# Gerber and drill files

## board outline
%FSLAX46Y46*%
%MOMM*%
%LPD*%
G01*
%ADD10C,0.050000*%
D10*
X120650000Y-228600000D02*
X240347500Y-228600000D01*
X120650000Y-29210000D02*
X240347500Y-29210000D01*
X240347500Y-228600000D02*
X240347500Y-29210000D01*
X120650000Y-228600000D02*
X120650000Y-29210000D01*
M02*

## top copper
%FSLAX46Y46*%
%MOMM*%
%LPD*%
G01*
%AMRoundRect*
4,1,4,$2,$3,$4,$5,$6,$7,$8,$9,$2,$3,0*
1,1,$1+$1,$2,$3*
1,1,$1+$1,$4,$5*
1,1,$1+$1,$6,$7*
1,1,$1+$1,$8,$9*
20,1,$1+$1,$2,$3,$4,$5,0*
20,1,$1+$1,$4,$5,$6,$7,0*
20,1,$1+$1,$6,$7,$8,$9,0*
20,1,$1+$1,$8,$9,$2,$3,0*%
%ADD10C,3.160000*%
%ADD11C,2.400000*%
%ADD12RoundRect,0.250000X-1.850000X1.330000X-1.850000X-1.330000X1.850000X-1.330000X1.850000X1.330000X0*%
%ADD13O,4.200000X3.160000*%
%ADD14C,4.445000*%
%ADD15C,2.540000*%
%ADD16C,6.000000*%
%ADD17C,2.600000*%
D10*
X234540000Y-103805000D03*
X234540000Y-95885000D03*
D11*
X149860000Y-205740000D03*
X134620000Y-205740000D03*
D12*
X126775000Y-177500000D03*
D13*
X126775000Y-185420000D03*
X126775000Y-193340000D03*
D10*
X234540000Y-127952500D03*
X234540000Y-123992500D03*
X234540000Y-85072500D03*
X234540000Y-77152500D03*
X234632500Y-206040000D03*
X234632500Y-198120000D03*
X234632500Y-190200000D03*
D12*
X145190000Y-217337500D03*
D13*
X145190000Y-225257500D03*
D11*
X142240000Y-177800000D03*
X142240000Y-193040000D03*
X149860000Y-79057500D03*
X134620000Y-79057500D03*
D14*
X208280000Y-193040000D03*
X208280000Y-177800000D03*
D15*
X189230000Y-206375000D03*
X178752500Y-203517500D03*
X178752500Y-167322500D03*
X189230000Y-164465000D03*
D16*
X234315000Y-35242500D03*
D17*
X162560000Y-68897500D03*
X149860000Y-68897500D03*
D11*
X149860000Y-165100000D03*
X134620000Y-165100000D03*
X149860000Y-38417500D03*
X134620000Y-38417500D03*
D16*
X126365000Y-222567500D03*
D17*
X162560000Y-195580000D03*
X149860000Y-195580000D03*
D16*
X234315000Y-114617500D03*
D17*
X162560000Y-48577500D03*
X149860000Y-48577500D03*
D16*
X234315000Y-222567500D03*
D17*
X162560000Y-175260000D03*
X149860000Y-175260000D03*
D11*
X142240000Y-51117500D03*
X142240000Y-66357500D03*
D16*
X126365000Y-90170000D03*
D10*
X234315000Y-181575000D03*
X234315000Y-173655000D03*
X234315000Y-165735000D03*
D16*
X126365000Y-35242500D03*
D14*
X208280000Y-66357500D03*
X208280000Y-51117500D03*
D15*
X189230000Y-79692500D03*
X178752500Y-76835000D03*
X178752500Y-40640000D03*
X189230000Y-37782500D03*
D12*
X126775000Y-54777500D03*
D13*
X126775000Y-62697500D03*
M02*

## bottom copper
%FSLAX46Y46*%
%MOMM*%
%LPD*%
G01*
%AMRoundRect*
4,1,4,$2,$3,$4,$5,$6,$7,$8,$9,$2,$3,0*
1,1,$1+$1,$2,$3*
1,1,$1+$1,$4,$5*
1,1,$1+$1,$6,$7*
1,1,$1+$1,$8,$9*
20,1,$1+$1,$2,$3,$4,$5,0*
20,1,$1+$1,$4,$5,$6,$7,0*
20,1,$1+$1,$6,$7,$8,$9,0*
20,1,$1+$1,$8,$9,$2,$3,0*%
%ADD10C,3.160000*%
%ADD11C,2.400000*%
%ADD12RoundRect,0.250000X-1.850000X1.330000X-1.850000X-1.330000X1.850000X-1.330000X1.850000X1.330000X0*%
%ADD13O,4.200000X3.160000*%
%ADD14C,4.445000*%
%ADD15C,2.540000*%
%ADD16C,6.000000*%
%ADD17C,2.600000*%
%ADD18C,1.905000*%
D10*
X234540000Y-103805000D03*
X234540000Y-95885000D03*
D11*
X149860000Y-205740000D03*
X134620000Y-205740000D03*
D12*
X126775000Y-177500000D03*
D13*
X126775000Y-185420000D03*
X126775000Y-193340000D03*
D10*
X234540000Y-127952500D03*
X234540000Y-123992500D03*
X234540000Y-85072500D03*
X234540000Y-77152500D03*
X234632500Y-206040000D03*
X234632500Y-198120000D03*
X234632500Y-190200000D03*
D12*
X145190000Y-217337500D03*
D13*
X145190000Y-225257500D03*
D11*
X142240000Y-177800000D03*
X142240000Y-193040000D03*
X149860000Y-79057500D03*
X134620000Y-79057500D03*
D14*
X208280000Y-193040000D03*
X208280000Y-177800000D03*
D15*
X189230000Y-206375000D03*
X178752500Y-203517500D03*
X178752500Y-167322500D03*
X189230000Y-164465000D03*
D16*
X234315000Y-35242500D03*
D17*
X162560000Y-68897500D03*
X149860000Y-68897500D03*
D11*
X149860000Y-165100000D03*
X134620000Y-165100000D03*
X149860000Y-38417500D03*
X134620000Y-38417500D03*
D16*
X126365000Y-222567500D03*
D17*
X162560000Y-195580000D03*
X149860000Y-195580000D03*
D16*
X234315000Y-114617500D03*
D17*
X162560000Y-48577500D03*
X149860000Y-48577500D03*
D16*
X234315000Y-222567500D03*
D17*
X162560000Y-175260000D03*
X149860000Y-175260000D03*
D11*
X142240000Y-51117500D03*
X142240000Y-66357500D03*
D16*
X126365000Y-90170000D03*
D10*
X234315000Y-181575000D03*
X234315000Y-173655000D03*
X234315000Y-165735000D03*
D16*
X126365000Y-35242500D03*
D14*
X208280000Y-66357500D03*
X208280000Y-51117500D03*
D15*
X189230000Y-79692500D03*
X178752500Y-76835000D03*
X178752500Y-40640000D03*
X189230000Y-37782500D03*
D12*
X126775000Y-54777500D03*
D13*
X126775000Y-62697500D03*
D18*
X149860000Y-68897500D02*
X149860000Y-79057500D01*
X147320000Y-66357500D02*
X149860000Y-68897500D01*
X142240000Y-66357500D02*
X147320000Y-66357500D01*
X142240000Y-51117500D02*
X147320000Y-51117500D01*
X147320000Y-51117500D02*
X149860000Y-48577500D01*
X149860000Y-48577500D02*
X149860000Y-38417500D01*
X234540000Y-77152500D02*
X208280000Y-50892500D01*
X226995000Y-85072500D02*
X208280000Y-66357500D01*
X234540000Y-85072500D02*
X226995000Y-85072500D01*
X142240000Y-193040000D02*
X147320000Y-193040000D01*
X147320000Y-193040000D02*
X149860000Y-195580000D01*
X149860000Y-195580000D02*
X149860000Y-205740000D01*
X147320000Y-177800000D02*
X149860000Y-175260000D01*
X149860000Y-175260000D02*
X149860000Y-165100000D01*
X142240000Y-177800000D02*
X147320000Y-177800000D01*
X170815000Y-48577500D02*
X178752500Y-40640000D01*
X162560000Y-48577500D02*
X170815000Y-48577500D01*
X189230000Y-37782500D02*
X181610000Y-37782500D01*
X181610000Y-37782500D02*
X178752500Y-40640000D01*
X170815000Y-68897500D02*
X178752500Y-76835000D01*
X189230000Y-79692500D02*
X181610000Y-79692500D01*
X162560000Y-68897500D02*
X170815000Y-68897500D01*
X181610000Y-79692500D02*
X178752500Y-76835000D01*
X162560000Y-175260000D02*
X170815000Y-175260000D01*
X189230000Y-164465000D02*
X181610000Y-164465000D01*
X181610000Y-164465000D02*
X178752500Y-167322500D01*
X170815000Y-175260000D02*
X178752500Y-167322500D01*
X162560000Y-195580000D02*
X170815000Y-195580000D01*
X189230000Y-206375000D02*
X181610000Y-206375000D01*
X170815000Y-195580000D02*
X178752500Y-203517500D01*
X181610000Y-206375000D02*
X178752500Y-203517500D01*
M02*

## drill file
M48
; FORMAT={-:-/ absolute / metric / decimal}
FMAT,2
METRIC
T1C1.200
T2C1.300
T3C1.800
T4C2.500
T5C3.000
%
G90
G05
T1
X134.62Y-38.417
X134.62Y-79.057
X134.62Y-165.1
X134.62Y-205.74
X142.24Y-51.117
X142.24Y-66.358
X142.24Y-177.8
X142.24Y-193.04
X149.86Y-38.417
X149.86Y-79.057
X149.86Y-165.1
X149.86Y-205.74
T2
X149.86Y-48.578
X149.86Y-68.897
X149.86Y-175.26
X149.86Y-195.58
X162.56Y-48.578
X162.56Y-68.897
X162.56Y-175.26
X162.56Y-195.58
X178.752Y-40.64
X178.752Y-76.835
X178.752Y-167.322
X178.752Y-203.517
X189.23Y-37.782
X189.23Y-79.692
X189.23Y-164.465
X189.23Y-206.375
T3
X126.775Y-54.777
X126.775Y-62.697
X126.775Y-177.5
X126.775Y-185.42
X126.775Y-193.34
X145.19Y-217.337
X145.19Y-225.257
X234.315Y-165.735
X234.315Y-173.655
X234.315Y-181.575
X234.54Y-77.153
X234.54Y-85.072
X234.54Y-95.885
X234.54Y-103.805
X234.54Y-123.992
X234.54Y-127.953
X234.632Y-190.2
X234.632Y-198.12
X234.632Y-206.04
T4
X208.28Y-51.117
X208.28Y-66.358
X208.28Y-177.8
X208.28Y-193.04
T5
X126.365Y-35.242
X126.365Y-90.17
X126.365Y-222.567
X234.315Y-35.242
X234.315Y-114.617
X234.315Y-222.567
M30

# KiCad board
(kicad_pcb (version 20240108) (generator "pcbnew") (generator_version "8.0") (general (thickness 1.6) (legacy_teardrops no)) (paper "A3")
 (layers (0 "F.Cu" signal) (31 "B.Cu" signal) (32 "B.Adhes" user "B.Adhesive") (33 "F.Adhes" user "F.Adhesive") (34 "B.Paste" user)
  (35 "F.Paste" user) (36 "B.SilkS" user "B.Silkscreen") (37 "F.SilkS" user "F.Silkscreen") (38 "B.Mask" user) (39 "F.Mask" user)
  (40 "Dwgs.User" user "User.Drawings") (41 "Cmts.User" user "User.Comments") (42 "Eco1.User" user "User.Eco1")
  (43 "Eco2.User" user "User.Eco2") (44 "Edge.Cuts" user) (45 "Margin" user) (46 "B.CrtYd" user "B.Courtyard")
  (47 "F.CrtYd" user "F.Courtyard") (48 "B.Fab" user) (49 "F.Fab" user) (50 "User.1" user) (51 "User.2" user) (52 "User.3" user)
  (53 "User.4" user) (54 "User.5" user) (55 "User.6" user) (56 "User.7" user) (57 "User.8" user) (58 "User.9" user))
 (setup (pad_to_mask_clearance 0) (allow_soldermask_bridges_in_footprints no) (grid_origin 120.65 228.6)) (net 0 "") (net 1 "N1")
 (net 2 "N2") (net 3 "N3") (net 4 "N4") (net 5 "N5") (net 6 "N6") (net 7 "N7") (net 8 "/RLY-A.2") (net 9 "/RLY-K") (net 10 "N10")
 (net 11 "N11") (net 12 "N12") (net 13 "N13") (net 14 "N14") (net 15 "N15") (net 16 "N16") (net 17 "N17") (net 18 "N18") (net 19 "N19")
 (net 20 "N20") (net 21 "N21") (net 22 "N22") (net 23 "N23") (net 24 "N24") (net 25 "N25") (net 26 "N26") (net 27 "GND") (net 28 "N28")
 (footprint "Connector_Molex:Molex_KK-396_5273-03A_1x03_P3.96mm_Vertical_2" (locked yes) (layer "F.Cu") (at 234.54 103.805 90)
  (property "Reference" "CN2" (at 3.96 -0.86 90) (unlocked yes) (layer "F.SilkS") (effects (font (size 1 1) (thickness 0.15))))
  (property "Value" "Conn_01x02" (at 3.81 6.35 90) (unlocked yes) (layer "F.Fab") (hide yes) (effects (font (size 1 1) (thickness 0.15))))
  (pad "1" thru_hole circle (at 0 0 90) (size 3.16 3.16) (drill 1.8) (layers "*.Cu" "*.Mask") (remove_unused_layers no) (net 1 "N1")
   (thermal_bridge_angle 90))
  (pad "2" thru_hole circle (at 7.92 0 90) (size 3.16 3.16) (drill 1.8) (layers "*.Cu" "*.Mask") (remove_unused_layers no) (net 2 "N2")
   (thermal_bridge_angle 90)))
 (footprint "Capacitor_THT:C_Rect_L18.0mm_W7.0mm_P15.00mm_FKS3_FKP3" (layer "F.Cu") (at 142.24 205.74 180)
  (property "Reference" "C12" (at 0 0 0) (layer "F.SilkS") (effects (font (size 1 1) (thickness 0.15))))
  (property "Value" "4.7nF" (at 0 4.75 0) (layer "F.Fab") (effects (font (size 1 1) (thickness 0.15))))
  (pad "1" thru_hole circle (at -7.62 0 180) (size 2.4 2.4) (drill 1.2) (layers "*.Cu" "*.Mask") (remove_unused_layers no) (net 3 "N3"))
  (pad "2" thru_hole circle (at 7.62 0 180) (size 2.4 2.4) (drill 1.2) (layers "*.Cu" "*.Mask") (remove_unused_layers no) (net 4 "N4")))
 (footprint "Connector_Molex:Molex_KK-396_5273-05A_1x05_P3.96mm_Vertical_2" (layer "F.Cu") (at 126.775 177.5 -90)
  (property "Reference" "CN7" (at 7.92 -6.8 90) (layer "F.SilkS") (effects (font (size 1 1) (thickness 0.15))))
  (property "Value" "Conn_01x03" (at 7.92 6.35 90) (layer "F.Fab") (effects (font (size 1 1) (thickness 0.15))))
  (pad "1" thru_hole roundrect (at 0 0 270) (size 3.16 4.2) (drill 1.8) (layers "*.Cu" "*.Mask") (remove_unused_layers no)
   (roundrect_rratio 0.079114) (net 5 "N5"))
  (pad "2" thru_hole oval (at 7.92 0 270) (size 3.16 4.2) (drill 1.8) (layers "*.Cu" "*.Mask") (remove_unused_layers no) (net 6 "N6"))
  (pad "3" thru_hole oval (at 15.84 0 270) (size 3.16 4.2) (drill 1.8) (layers "*.Cu" "*.Mask") (remove_unused_layers no) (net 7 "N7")))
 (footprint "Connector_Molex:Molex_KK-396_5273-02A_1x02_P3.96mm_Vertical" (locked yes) (layer "F.Cu") (at 234.54 127.9525 90)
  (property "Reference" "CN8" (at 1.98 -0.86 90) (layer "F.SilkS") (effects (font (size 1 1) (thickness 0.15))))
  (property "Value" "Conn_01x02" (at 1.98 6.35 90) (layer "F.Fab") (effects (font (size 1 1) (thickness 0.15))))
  (pad "1" thru_hole circle (at 0 0 90) (size 3.16 3.16) (drill 1.8) (layers "*.Cu" "*.Mask") (remove_unused_layers no) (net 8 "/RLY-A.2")
   (thermal_bridge_angle 90))
  (pad "2" thru_hole circle (at 3.96 0 90) (size 3.16 3.16) (drill 1.8) (layers "*.Cu" "*.Mask") (remove_unused_layers no) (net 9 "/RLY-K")
   (thermal_bridge_angle 90)))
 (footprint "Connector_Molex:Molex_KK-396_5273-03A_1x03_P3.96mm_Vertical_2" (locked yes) (layer "F.Cu") (at 234.54 85.0725 90)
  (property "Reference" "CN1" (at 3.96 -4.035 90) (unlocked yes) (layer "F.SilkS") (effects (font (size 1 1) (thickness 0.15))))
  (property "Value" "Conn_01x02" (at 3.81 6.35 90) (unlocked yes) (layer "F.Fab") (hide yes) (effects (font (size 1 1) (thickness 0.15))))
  (pad "1" thru_hole circle (at 0 0 90) (size 3.16 4.2) (drill 1.8) (layers "*.Cu" "*.Mask") (remove_unused_layers no) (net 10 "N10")
   (thermal_bridge_angle 90))
  (pad "2" thru_hole circle (at 7.92 0 90) (size 3.16 4.2) (drill 1.8) (layers "*.Cu" "*.Mask") (remove_unused_layers no) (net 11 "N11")
   (thermal_bridge_angle 90)))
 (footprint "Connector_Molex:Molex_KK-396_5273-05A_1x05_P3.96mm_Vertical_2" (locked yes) (layer "F.Cu") (at 234.6325 206.04 90)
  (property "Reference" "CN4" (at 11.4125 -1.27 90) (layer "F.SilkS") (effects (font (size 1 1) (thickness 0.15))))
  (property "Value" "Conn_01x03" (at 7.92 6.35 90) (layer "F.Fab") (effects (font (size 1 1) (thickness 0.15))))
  (pad "1" thru_hole circle (at 0 0 90) (size 3.16 4.2) (drill 1.8) (layers "*.Cu" "*.Mask") (remove_unused_layers no) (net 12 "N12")
   (thermal_bridge_angle 90))
  (pad "2" thru_hole circle (at 7.92 0 90) (size 3.16 4.2) (drill 1.8) (layers "*.Cu" "*.Mask") (remove_unused_layers no) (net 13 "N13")
   (thermal_bridge_angle 90))
  (pad "3" thru_hole circle (at 15.84 0 90) (size 3.16 4.2) (drill 1.8) (layers "*.Cu" "*.Mask") (remove_unused_layers no) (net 4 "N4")
   (thermal_bridge_angle 90)))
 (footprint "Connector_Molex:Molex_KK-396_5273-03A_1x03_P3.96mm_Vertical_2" (layer "F.Cu") (at 145.19 217.3375 -90)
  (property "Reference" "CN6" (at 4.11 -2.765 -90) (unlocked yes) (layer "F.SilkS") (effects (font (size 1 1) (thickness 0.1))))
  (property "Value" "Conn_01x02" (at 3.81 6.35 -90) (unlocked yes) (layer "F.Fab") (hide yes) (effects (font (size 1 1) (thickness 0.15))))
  (pad "1" thru_hole roundrect (at 0 0 270) (size 3.16 4.2) (drill 1.8) (layers "*.Cu" "*.Mask") (remove_unused_layers no)
   (roundrect_rratio 0.079114) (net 13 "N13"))
  (pad "2" thru_hole oval (at 7.92 0 270) (size 3.16 4.2) (drill 1.8) (layers "*.Cu" "*.Mask") (remove_unused_layers no) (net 12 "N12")))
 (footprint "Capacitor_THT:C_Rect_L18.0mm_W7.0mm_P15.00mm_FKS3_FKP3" (layer "F.Cu") (at 142.24 185.42 -90)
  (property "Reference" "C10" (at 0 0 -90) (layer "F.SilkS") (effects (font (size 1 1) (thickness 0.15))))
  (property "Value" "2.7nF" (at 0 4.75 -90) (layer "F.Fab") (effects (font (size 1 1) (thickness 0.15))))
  (pad "1" thru_hole circle (at -7.62 0 270) (size 2.4 2.4) (drill 1.2) (layers "*.Cu" "*.Mask") (remove_unused_layers no) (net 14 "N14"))
  (pad "2" thru_hole circle (at 7.62 0 270) (size 2.4 2.4) (drill 1.2) (layers "*.Cu" "*.Mask") (remove_unused_layers no) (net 3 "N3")))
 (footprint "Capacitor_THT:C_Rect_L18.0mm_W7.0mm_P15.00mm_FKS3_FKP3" (layer "F.Cu") (at 142.24 79.0575 180)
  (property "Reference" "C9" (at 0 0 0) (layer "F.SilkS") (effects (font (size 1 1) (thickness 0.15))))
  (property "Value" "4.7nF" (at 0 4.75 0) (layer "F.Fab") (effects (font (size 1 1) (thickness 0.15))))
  (pad "1" thru_hole circle (at -7.62 0 180) (size 2.4 2.4) (drill 1.2) (layers "*.Cu" "*.Mask") (remove_unused_layers no) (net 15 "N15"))
  (pad "2" thru_hole circle (at 7.62 0 180) (size 2.4 2.4) (drill 1.2) (layers "*.Cu" "*.Mask") (remove_unused_layers no) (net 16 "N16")))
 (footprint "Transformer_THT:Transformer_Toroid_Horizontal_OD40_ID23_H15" (layer "F.Cu") (at 189.23 185.42 90)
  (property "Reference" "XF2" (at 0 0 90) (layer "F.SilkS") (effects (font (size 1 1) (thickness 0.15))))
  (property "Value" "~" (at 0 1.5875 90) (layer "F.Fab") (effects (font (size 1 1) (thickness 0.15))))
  (pad "1" thru_hole circle (at -7.62 19.05 90) (size 4.445 2.54) (drill 2.5) (layers "*.Cu" "*.Mask") (remove_unused_layers no)
   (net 1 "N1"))
  (pad "2" thru_hole circle (at 7.62 19.05 90) (size 4.445 2.54) (drill 2.5) (layers "*.Cu" "*.Mask") (remove_unused_layers no) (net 2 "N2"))
  (pad "3" thru_hole circle (at -20.955 0 90) (size 2.54 2.54) (drill 1.3) (layers "*.Cu" "*.Mask") (remove_unused_layers no) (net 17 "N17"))
  (pad "3" thru_hole circle (at -18.0975 -10.4775 90) (size 2.54 2.54) (drill 1.3) (layers "*.Cu" "*.Mask") (remove_unused_layers no)
   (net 17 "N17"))
  (pad "4" thru_hole circle (at 18.0975 -10.4775 90) (size 2.54 2.54) (drill 1.3) (layers "*.Cu" "*.Mask") (remove_unused_layers no)
   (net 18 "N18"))
  (pad "4" thru_hole circle (at 20.955 0 90) (size 2.54 2.54) (drill 1.3) (layers "*.Cu" "*.Mask") (remove_unused_layers no) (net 18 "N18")))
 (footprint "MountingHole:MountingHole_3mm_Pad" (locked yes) (layer "F.Cu") (at 234.315 35.2425 -90)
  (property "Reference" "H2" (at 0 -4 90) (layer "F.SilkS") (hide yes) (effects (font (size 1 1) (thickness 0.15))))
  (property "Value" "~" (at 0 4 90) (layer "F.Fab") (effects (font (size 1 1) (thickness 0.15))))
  (pad "1" thru_hole circle (at 0 0 270) (size 6 6) (drill 3) (layers "*.Cu" "*.Mask") (remove_unused_layers no) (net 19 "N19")))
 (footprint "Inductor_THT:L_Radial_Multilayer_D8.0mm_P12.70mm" (layer "F.Cu") (at 158.115 68.8975 180)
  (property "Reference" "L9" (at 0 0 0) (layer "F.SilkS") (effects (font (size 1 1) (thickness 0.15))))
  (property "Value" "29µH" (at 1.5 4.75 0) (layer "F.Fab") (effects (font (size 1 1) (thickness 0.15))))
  (pad "1" thru_hole circle (at -4.445 0 180) (size 2.6 2.6) (drill 1.3) (layers "*.Cu" "*.Mask") (remove_unused_layers no) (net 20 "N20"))
  (pad "2" thru_hole circle (at 8.255 0 180) (size 2.6 2.6) (drill 1.3) (layers "*.Cu" "*.Mask") (remove_unused_layers no) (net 15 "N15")))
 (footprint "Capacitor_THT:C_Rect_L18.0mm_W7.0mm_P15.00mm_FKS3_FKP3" (layer "F.Cu") (at 142.24 165.1 180)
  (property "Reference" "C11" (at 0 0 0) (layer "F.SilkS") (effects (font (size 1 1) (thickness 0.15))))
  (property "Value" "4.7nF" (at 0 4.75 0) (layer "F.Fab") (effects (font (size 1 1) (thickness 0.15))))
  (pad "1" thru_hole circle (at -7.62 0 180) (size 2.4 2.4) (drill 1.2) (layers "*.Cu" "*.Mask") (remove_unused_layers no) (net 14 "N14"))
  (pad "2" thru_hole circle (at 7.62 0 180) (size 2.4 2.4) (drill 1.2) (layers "*.Cu" "*.Mask") (remove_unused_layers no) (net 7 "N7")))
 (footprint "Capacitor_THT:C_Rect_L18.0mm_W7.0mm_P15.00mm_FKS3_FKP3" (layer "F.Cu") (at 142.24 38.4175 180)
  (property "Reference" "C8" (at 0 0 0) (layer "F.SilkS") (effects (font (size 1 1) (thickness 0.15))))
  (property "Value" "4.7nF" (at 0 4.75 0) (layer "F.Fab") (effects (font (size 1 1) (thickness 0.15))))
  (pad "1" thru_hole circle (at -7.62 0 180) (size 2.4 2.4) (drill 1.2) (layers "*.Cu" "*.Mask") (remove_unused_layers no) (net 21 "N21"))
  (pad "2" thru_hole circle (at 7.62 0 180) (size 2.4 2.4) (drill 1.2) (layers "*.Cu" "*.Mask") (remove_unused_layers no) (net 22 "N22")))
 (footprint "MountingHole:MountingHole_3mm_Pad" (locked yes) (layer "F.Cu") (at 126.365 222.5675)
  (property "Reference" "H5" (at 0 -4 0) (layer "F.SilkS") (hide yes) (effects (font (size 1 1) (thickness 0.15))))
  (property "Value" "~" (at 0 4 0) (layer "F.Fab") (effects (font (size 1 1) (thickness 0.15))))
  (pad "1" thru_hole circle (at 0 0) (size 6 6) (drill 3) (layers "*.Cu" "*.Mask") (remove_unused_layers no) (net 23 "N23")))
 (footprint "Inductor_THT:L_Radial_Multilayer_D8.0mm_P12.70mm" (layer "F.Cu") (at 158.115 195.58 180)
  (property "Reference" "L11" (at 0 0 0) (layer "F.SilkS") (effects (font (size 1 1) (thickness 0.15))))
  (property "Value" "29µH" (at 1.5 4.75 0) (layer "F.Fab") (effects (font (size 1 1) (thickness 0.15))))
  (pad "1" thru_hole circle (at -4.445 0 180) (size 2.6 2.6) (drill 1.3) (layers "*.Cu" "*.Mask") (remove_unused_layers no) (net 17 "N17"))
  (pad "2" thru_hole circle (at 8.255 0 180) (size 2.6 2.6) (drill 1.3) (layers "*.Cu" "*.Mask") (remove_unused_layers no) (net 3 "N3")))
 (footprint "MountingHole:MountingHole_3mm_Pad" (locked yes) (layer "F.Cu") (at 234.315 114.6175 -90)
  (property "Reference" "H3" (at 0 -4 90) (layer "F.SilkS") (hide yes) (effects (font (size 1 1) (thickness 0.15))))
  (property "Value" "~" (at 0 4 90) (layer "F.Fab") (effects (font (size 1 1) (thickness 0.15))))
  (pad "1" thru_hole circle (at 0 0 270) (size 6 6) (drill 3) (layers "*.Cu" "*.Mask") (remove_unused_layers no) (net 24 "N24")))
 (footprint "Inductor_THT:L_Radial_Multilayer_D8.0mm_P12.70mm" (layer "F.Cu") (at 158.115 48.5775 180)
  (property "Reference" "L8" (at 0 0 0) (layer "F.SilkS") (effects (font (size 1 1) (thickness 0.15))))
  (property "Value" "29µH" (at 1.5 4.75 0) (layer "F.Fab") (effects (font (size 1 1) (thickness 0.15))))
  (pad "1" thru_hole circle (at -4.445 0 180) (size 2.6 2.6) (drill 1.3) (layers "*.Cu" "*.Mask") (remove_unused_layers no) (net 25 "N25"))
  (pad "2" thru_hole circle (at 8.255 0 180) (size 2.6 2.6) (drill 1.3) (layers "*.Cu" "*.Mask") (remove_unused_layers no) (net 21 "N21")))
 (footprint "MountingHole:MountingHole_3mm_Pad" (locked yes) (layer "F.Cu") (at 234.315 222.5675)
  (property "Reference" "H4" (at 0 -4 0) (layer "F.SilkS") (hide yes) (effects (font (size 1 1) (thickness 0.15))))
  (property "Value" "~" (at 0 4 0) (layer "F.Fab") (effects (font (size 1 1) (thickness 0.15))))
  (pad "1" thru_hole circle (at 0 0) (size 6 6) (drill 3) (layers "*.Cu" "*.Mask") (remove_unused_layers no) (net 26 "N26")))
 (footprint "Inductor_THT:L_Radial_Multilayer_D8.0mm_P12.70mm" (layer "F.Cu") (at 158.115 175.26 180)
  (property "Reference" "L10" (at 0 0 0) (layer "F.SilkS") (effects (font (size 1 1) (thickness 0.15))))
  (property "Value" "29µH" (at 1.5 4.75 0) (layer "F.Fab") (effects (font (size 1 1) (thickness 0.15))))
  (pad "1" thru_hole circle (at -4.445 0 180) (size 2.6 2.6) (drill 1.3) (layers "*.Cu" "*.Mask") (remove_unused_layers no) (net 18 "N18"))
  (pad "2" thru_hole circle (at 8.255 0 180) (size 2.6 2.6) (drill 1.3) (layers "*.Cu" "*.Mask") (remove_unused_layers no) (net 14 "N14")))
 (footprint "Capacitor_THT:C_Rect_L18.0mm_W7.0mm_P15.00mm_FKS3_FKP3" (layer "F.Cu") (at 142.24 58.7375 -90)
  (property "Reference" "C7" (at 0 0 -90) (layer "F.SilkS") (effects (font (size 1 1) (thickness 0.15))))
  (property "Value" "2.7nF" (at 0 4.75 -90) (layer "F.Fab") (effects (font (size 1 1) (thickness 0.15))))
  (pad "1" thru_hole circle (at -7.62 0 270) (size 2.4 2.4) (drill 1.2) (layers "*.Cu" "*.Mask") (remove_unused_layers no) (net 21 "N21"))
  (pad "2" thru_hole circle (at 7.62 0 270) (size 2.4 2.4) (drill 1.2) (layers "*.Cu" "*.Mask") (remove_unused_layers no) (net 15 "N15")))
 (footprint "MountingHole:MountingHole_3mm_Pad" (layer "F.Cu") (at 126.365 90.17)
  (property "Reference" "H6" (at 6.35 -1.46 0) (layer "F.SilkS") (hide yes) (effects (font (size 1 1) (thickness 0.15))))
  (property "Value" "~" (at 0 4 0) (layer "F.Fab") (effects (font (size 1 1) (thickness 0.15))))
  (pad "1" thru_hole circle (at 0 0) (size 6 6) (drill 3) (layers "*.Cu" "*.Mask") (remove_unused_layers no) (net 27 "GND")))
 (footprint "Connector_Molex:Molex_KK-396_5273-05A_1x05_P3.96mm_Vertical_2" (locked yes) (layer "F.Cu") (at 234.315 181.575 90)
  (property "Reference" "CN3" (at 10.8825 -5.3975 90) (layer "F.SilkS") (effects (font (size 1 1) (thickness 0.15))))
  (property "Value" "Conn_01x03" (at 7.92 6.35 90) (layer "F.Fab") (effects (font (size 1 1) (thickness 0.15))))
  (pad "1" thru_hole circle (at 0 0 90) (size 3.16 4.2) (drill 1.8) (layers "*.Cu" "*.Mask") (remove_unused_layers no) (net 7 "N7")
   (thermal_bridge_angle 90))
  (pad "2" thru_hole circle (at 7.92 0 90) (size 3.16 4.2) (drill 1.8) (layers "*.Cu" "*.Mask") (remove_unused_layers no) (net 6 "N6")
   (thermal_bridge_angle 90))
  (pad "3" thru_hole circle (at 15.84 0 90) (size 3.16 4.2) (drill 1.8) (layers "*.Cu" "*.Mask") (remove_unused_layers no) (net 5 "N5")
   (thermal_bridge_angle 90)))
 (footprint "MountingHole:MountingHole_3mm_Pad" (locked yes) (layer "F.Cu") (at 126.365 35.2425)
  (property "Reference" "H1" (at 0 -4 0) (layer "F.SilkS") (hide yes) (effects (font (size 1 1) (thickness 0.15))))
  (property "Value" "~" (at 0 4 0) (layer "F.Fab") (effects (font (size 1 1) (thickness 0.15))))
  (pad "1" thru_hole circle (at 0 0) (size 6 6) (drill 3) (layers "*.Cu" "*.Mask") (remove_unused_layers no) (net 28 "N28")))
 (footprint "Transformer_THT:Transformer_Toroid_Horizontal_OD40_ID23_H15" (layer "F.Cu") (at 189.23 58.7375 90)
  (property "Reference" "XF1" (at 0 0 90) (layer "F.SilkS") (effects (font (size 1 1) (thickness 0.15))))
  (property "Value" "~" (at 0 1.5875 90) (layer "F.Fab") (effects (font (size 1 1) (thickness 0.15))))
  (pad "1" thru_hole circle (at -7.62 19.05 90) (size 4.445 2.54) (drill 2.5) (layers "*.Cu" "*.Mask") (remove_unused_layers no)
   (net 10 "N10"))
  (pad "2" thru_hole circle (at 7.62 19.05 90) (size 4.445 2.54) (drill 2.5) (layers "*.Cu" "*.Mask") (remove_unused_layers no)
   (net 11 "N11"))
  (pad "3" thru_hole circle (at -20.955 0 90) (size 2.54 2.54) (drill 1.3) (layers "*.Cu" "*.Mask") (remove_unused_layers no) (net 20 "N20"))
  (pad "3" thru_hole circle (at -18.0975 -10.4775 90) (size 2.54 2.54) (drill 1.3) (layers "*.Cu" "*.Mask") (remove_unused_layers no)
   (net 20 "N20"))
  (pad "4" thru_hole circle (at 18.0975 -10.4775 90) (size 2.54 2.54) (drill 1.3) (layers "*.Cu" "*.Mask") (remove_unused_layers no)
   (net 25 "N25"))
  (pad "4" thru_hole circle (at 20.955 0 90) (size 2.54 2.54) (drill 1.3) (layers "*.Cu" "*.Mask") (remove_unused_layers no) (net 25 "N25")))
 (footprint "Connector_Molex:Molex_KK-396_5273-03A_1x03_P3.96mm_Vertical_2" (layer "F.Cu") (at 126.775 54.7775 -90)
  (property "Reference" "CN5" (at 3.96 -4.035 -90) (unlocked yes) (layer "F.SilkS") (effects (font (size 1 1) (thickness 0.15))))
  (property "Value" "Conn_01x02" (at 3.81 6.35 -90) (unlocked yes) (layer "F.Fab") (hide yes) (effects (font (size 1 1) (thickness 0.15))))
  (pad "1" thru_hole roundrect (at 0 0 270) (size 3.16 4.2) (drill 1.8) (layers "*.Cu" "*.Mask") (remove_unused_layers no)
   (roundrect_rratio 0.079114) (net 22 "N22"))
  (pad "2" thru_hole oval (at 7.92 0 270) (size 3.16 4.2) (drill 1.8) (layers "*.Cu" "*.Mask") (remove_unused_layers no) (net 16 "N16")))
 (gr_line (start 120.65 228.6) (end 240.3475 228.6) (locked yes) (stroke (width 0.05) (type default)) (layer "Edge.Cuts"))
 (gr_line (start 120.65 29.21) (end 240.3475 29.21) (locked yes) (stroke (width 0.05) (type default)) (layer "Edge.Cuts"))
 (gr_line (start 240.3475 228.6) (end 240.3475 29.21) (locked yes) (stroke (width 0.05) (type default)) (layer "Edge.Cuts"))
 (gr_line (start 120.65 228.6) (end 120.65 29.21) (locked yes) (stroke (width 0.05) (type default)) (layer "Edge.Cuts"))
 (segment (start 149.86 68.8975) (end 149.86 79.0575) (width 1.905) (layer "B.Cu") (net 15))
 (segment (start 147.32 66.3575) (end 149.86 68.8975) (width 1.905) (layer "B.Cu") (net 15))
 (segment (start 142.24 66.3575) (end 147.32 66.3575) (width 1.905) (layer "B.Cu") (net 15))
 (segment (start 142.24 51.1175) (end 147.32 51.1175) (width 1.905) (layer "B.Cu") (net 21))
 (segment (start 147.32 51.1175) (end 149.86 48.5775) (width 1.905) (layer "B.Cu") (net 21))
 (segment (start 149.86 48.5775) (end 149.86 38.4175) (width 1.905) (layer "B.Cu") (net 21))
 (segment (start 234.54 77.1525) (end 208.28 50.8925) (width 1.905) (layer "B.Cu") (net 11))
 (segment (start 226.995 85.0725) (end 208.28 66.3575) (width 1.905) (layer "B.Cu") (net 10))
 (segment (start 234.54 85.0725) (end 226.995 85.0725) (width 1.905) (layer "B.Cu") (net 10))
 (segment (start 142.24 193.04) (end 147.32 193.04) (width 1.905) (layer "B.Cu") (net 3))
 (segment (start 147.32 193.04) (end 149.86 195.58) (width 1.905) (layer "B.Cu") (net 3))
 (segment (start 149.86 195.58) (end 149.86 205.74) (width 1.905) (layer "B.Cu") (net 3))
 (segment (start 147.32 177.8) (end 149.86 175.26) (width 1.905) (layer "B.Cu") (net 14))
 (segment (start 149.86 175.26) (end 149.86 165.1) (width 1.905) (layer "B.Cu") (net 14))
 (segment (start 142.24 177.8) (end 147.32 177.8) (width 1.905) (layer "B.Cu") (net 14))
 (segment (start 170.815 48.5775) (end 178.7525 40.64) (width 1.905) (layer "B.Cu") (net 25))
 (segment (start 162.56 48.5775) (end 170.815 48.5775) (width 1.905) (layer "B.Cu") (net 25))
 (segment (start 189.23 37.7825) (end 181.61 37.7825) (width 1.905) (layer "B.Cu") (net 25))
 (segment (start 181.61 37.7825) (end 178.7525 40.64) (width 1.905) (layer "B.Cu") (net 25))
 (segment (start 170.815 68.8975) (end 178.7525 76.835) (width 1.905) (layer "B.Cu") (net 20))
 (segment (start 189.23 79.6925) (end 181.61 79.6925) (width 1.905) (layer "B.Cu") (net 20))
 (segment (start 162.56 68.8975) (end 170.815 68.8975) (width 1.905) (layer "B.Cu") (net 20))
 (segment (start 181.61 79.6925) (end 178.7525 76.835) (width 1.905) (layer "B.Cu") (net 20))
 (segment (start 162.56 175.26) (end 170.815 175.26) (width 1.905) (layer "B.Cu") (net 18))
 (segment (start 189.23 164.465) (end 181.61 164.465) (width 1.905) (layer "B.Cu") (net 18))
 (segment (start 181.61 164.465) (end 178.7525 167.3225) (width 1.905) (layer "B.Cu") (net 18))
 (segment (start 170.815 175.26) (end 178.7525 167.3225) (width 1.905) (layer "B.Cu") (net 18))
 (segment (start 162.56 195.58) (end 170.815 195.58) (width 1.905) (layer "B.Cu") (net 17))
 (segment (start 189.23 206.375) (end 181.61 206.375) (width 1.905) (layer "B.Cu") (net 17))
 (segment (start 170.815 195.58) (end 178.7525 203.5175) (width 1.905) (layer "B.Cu") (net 17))
 (segment (start 181.61 206.375) (end 178.7525 203.5175) (width 1.905) (layer "B.Cu") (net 17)))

